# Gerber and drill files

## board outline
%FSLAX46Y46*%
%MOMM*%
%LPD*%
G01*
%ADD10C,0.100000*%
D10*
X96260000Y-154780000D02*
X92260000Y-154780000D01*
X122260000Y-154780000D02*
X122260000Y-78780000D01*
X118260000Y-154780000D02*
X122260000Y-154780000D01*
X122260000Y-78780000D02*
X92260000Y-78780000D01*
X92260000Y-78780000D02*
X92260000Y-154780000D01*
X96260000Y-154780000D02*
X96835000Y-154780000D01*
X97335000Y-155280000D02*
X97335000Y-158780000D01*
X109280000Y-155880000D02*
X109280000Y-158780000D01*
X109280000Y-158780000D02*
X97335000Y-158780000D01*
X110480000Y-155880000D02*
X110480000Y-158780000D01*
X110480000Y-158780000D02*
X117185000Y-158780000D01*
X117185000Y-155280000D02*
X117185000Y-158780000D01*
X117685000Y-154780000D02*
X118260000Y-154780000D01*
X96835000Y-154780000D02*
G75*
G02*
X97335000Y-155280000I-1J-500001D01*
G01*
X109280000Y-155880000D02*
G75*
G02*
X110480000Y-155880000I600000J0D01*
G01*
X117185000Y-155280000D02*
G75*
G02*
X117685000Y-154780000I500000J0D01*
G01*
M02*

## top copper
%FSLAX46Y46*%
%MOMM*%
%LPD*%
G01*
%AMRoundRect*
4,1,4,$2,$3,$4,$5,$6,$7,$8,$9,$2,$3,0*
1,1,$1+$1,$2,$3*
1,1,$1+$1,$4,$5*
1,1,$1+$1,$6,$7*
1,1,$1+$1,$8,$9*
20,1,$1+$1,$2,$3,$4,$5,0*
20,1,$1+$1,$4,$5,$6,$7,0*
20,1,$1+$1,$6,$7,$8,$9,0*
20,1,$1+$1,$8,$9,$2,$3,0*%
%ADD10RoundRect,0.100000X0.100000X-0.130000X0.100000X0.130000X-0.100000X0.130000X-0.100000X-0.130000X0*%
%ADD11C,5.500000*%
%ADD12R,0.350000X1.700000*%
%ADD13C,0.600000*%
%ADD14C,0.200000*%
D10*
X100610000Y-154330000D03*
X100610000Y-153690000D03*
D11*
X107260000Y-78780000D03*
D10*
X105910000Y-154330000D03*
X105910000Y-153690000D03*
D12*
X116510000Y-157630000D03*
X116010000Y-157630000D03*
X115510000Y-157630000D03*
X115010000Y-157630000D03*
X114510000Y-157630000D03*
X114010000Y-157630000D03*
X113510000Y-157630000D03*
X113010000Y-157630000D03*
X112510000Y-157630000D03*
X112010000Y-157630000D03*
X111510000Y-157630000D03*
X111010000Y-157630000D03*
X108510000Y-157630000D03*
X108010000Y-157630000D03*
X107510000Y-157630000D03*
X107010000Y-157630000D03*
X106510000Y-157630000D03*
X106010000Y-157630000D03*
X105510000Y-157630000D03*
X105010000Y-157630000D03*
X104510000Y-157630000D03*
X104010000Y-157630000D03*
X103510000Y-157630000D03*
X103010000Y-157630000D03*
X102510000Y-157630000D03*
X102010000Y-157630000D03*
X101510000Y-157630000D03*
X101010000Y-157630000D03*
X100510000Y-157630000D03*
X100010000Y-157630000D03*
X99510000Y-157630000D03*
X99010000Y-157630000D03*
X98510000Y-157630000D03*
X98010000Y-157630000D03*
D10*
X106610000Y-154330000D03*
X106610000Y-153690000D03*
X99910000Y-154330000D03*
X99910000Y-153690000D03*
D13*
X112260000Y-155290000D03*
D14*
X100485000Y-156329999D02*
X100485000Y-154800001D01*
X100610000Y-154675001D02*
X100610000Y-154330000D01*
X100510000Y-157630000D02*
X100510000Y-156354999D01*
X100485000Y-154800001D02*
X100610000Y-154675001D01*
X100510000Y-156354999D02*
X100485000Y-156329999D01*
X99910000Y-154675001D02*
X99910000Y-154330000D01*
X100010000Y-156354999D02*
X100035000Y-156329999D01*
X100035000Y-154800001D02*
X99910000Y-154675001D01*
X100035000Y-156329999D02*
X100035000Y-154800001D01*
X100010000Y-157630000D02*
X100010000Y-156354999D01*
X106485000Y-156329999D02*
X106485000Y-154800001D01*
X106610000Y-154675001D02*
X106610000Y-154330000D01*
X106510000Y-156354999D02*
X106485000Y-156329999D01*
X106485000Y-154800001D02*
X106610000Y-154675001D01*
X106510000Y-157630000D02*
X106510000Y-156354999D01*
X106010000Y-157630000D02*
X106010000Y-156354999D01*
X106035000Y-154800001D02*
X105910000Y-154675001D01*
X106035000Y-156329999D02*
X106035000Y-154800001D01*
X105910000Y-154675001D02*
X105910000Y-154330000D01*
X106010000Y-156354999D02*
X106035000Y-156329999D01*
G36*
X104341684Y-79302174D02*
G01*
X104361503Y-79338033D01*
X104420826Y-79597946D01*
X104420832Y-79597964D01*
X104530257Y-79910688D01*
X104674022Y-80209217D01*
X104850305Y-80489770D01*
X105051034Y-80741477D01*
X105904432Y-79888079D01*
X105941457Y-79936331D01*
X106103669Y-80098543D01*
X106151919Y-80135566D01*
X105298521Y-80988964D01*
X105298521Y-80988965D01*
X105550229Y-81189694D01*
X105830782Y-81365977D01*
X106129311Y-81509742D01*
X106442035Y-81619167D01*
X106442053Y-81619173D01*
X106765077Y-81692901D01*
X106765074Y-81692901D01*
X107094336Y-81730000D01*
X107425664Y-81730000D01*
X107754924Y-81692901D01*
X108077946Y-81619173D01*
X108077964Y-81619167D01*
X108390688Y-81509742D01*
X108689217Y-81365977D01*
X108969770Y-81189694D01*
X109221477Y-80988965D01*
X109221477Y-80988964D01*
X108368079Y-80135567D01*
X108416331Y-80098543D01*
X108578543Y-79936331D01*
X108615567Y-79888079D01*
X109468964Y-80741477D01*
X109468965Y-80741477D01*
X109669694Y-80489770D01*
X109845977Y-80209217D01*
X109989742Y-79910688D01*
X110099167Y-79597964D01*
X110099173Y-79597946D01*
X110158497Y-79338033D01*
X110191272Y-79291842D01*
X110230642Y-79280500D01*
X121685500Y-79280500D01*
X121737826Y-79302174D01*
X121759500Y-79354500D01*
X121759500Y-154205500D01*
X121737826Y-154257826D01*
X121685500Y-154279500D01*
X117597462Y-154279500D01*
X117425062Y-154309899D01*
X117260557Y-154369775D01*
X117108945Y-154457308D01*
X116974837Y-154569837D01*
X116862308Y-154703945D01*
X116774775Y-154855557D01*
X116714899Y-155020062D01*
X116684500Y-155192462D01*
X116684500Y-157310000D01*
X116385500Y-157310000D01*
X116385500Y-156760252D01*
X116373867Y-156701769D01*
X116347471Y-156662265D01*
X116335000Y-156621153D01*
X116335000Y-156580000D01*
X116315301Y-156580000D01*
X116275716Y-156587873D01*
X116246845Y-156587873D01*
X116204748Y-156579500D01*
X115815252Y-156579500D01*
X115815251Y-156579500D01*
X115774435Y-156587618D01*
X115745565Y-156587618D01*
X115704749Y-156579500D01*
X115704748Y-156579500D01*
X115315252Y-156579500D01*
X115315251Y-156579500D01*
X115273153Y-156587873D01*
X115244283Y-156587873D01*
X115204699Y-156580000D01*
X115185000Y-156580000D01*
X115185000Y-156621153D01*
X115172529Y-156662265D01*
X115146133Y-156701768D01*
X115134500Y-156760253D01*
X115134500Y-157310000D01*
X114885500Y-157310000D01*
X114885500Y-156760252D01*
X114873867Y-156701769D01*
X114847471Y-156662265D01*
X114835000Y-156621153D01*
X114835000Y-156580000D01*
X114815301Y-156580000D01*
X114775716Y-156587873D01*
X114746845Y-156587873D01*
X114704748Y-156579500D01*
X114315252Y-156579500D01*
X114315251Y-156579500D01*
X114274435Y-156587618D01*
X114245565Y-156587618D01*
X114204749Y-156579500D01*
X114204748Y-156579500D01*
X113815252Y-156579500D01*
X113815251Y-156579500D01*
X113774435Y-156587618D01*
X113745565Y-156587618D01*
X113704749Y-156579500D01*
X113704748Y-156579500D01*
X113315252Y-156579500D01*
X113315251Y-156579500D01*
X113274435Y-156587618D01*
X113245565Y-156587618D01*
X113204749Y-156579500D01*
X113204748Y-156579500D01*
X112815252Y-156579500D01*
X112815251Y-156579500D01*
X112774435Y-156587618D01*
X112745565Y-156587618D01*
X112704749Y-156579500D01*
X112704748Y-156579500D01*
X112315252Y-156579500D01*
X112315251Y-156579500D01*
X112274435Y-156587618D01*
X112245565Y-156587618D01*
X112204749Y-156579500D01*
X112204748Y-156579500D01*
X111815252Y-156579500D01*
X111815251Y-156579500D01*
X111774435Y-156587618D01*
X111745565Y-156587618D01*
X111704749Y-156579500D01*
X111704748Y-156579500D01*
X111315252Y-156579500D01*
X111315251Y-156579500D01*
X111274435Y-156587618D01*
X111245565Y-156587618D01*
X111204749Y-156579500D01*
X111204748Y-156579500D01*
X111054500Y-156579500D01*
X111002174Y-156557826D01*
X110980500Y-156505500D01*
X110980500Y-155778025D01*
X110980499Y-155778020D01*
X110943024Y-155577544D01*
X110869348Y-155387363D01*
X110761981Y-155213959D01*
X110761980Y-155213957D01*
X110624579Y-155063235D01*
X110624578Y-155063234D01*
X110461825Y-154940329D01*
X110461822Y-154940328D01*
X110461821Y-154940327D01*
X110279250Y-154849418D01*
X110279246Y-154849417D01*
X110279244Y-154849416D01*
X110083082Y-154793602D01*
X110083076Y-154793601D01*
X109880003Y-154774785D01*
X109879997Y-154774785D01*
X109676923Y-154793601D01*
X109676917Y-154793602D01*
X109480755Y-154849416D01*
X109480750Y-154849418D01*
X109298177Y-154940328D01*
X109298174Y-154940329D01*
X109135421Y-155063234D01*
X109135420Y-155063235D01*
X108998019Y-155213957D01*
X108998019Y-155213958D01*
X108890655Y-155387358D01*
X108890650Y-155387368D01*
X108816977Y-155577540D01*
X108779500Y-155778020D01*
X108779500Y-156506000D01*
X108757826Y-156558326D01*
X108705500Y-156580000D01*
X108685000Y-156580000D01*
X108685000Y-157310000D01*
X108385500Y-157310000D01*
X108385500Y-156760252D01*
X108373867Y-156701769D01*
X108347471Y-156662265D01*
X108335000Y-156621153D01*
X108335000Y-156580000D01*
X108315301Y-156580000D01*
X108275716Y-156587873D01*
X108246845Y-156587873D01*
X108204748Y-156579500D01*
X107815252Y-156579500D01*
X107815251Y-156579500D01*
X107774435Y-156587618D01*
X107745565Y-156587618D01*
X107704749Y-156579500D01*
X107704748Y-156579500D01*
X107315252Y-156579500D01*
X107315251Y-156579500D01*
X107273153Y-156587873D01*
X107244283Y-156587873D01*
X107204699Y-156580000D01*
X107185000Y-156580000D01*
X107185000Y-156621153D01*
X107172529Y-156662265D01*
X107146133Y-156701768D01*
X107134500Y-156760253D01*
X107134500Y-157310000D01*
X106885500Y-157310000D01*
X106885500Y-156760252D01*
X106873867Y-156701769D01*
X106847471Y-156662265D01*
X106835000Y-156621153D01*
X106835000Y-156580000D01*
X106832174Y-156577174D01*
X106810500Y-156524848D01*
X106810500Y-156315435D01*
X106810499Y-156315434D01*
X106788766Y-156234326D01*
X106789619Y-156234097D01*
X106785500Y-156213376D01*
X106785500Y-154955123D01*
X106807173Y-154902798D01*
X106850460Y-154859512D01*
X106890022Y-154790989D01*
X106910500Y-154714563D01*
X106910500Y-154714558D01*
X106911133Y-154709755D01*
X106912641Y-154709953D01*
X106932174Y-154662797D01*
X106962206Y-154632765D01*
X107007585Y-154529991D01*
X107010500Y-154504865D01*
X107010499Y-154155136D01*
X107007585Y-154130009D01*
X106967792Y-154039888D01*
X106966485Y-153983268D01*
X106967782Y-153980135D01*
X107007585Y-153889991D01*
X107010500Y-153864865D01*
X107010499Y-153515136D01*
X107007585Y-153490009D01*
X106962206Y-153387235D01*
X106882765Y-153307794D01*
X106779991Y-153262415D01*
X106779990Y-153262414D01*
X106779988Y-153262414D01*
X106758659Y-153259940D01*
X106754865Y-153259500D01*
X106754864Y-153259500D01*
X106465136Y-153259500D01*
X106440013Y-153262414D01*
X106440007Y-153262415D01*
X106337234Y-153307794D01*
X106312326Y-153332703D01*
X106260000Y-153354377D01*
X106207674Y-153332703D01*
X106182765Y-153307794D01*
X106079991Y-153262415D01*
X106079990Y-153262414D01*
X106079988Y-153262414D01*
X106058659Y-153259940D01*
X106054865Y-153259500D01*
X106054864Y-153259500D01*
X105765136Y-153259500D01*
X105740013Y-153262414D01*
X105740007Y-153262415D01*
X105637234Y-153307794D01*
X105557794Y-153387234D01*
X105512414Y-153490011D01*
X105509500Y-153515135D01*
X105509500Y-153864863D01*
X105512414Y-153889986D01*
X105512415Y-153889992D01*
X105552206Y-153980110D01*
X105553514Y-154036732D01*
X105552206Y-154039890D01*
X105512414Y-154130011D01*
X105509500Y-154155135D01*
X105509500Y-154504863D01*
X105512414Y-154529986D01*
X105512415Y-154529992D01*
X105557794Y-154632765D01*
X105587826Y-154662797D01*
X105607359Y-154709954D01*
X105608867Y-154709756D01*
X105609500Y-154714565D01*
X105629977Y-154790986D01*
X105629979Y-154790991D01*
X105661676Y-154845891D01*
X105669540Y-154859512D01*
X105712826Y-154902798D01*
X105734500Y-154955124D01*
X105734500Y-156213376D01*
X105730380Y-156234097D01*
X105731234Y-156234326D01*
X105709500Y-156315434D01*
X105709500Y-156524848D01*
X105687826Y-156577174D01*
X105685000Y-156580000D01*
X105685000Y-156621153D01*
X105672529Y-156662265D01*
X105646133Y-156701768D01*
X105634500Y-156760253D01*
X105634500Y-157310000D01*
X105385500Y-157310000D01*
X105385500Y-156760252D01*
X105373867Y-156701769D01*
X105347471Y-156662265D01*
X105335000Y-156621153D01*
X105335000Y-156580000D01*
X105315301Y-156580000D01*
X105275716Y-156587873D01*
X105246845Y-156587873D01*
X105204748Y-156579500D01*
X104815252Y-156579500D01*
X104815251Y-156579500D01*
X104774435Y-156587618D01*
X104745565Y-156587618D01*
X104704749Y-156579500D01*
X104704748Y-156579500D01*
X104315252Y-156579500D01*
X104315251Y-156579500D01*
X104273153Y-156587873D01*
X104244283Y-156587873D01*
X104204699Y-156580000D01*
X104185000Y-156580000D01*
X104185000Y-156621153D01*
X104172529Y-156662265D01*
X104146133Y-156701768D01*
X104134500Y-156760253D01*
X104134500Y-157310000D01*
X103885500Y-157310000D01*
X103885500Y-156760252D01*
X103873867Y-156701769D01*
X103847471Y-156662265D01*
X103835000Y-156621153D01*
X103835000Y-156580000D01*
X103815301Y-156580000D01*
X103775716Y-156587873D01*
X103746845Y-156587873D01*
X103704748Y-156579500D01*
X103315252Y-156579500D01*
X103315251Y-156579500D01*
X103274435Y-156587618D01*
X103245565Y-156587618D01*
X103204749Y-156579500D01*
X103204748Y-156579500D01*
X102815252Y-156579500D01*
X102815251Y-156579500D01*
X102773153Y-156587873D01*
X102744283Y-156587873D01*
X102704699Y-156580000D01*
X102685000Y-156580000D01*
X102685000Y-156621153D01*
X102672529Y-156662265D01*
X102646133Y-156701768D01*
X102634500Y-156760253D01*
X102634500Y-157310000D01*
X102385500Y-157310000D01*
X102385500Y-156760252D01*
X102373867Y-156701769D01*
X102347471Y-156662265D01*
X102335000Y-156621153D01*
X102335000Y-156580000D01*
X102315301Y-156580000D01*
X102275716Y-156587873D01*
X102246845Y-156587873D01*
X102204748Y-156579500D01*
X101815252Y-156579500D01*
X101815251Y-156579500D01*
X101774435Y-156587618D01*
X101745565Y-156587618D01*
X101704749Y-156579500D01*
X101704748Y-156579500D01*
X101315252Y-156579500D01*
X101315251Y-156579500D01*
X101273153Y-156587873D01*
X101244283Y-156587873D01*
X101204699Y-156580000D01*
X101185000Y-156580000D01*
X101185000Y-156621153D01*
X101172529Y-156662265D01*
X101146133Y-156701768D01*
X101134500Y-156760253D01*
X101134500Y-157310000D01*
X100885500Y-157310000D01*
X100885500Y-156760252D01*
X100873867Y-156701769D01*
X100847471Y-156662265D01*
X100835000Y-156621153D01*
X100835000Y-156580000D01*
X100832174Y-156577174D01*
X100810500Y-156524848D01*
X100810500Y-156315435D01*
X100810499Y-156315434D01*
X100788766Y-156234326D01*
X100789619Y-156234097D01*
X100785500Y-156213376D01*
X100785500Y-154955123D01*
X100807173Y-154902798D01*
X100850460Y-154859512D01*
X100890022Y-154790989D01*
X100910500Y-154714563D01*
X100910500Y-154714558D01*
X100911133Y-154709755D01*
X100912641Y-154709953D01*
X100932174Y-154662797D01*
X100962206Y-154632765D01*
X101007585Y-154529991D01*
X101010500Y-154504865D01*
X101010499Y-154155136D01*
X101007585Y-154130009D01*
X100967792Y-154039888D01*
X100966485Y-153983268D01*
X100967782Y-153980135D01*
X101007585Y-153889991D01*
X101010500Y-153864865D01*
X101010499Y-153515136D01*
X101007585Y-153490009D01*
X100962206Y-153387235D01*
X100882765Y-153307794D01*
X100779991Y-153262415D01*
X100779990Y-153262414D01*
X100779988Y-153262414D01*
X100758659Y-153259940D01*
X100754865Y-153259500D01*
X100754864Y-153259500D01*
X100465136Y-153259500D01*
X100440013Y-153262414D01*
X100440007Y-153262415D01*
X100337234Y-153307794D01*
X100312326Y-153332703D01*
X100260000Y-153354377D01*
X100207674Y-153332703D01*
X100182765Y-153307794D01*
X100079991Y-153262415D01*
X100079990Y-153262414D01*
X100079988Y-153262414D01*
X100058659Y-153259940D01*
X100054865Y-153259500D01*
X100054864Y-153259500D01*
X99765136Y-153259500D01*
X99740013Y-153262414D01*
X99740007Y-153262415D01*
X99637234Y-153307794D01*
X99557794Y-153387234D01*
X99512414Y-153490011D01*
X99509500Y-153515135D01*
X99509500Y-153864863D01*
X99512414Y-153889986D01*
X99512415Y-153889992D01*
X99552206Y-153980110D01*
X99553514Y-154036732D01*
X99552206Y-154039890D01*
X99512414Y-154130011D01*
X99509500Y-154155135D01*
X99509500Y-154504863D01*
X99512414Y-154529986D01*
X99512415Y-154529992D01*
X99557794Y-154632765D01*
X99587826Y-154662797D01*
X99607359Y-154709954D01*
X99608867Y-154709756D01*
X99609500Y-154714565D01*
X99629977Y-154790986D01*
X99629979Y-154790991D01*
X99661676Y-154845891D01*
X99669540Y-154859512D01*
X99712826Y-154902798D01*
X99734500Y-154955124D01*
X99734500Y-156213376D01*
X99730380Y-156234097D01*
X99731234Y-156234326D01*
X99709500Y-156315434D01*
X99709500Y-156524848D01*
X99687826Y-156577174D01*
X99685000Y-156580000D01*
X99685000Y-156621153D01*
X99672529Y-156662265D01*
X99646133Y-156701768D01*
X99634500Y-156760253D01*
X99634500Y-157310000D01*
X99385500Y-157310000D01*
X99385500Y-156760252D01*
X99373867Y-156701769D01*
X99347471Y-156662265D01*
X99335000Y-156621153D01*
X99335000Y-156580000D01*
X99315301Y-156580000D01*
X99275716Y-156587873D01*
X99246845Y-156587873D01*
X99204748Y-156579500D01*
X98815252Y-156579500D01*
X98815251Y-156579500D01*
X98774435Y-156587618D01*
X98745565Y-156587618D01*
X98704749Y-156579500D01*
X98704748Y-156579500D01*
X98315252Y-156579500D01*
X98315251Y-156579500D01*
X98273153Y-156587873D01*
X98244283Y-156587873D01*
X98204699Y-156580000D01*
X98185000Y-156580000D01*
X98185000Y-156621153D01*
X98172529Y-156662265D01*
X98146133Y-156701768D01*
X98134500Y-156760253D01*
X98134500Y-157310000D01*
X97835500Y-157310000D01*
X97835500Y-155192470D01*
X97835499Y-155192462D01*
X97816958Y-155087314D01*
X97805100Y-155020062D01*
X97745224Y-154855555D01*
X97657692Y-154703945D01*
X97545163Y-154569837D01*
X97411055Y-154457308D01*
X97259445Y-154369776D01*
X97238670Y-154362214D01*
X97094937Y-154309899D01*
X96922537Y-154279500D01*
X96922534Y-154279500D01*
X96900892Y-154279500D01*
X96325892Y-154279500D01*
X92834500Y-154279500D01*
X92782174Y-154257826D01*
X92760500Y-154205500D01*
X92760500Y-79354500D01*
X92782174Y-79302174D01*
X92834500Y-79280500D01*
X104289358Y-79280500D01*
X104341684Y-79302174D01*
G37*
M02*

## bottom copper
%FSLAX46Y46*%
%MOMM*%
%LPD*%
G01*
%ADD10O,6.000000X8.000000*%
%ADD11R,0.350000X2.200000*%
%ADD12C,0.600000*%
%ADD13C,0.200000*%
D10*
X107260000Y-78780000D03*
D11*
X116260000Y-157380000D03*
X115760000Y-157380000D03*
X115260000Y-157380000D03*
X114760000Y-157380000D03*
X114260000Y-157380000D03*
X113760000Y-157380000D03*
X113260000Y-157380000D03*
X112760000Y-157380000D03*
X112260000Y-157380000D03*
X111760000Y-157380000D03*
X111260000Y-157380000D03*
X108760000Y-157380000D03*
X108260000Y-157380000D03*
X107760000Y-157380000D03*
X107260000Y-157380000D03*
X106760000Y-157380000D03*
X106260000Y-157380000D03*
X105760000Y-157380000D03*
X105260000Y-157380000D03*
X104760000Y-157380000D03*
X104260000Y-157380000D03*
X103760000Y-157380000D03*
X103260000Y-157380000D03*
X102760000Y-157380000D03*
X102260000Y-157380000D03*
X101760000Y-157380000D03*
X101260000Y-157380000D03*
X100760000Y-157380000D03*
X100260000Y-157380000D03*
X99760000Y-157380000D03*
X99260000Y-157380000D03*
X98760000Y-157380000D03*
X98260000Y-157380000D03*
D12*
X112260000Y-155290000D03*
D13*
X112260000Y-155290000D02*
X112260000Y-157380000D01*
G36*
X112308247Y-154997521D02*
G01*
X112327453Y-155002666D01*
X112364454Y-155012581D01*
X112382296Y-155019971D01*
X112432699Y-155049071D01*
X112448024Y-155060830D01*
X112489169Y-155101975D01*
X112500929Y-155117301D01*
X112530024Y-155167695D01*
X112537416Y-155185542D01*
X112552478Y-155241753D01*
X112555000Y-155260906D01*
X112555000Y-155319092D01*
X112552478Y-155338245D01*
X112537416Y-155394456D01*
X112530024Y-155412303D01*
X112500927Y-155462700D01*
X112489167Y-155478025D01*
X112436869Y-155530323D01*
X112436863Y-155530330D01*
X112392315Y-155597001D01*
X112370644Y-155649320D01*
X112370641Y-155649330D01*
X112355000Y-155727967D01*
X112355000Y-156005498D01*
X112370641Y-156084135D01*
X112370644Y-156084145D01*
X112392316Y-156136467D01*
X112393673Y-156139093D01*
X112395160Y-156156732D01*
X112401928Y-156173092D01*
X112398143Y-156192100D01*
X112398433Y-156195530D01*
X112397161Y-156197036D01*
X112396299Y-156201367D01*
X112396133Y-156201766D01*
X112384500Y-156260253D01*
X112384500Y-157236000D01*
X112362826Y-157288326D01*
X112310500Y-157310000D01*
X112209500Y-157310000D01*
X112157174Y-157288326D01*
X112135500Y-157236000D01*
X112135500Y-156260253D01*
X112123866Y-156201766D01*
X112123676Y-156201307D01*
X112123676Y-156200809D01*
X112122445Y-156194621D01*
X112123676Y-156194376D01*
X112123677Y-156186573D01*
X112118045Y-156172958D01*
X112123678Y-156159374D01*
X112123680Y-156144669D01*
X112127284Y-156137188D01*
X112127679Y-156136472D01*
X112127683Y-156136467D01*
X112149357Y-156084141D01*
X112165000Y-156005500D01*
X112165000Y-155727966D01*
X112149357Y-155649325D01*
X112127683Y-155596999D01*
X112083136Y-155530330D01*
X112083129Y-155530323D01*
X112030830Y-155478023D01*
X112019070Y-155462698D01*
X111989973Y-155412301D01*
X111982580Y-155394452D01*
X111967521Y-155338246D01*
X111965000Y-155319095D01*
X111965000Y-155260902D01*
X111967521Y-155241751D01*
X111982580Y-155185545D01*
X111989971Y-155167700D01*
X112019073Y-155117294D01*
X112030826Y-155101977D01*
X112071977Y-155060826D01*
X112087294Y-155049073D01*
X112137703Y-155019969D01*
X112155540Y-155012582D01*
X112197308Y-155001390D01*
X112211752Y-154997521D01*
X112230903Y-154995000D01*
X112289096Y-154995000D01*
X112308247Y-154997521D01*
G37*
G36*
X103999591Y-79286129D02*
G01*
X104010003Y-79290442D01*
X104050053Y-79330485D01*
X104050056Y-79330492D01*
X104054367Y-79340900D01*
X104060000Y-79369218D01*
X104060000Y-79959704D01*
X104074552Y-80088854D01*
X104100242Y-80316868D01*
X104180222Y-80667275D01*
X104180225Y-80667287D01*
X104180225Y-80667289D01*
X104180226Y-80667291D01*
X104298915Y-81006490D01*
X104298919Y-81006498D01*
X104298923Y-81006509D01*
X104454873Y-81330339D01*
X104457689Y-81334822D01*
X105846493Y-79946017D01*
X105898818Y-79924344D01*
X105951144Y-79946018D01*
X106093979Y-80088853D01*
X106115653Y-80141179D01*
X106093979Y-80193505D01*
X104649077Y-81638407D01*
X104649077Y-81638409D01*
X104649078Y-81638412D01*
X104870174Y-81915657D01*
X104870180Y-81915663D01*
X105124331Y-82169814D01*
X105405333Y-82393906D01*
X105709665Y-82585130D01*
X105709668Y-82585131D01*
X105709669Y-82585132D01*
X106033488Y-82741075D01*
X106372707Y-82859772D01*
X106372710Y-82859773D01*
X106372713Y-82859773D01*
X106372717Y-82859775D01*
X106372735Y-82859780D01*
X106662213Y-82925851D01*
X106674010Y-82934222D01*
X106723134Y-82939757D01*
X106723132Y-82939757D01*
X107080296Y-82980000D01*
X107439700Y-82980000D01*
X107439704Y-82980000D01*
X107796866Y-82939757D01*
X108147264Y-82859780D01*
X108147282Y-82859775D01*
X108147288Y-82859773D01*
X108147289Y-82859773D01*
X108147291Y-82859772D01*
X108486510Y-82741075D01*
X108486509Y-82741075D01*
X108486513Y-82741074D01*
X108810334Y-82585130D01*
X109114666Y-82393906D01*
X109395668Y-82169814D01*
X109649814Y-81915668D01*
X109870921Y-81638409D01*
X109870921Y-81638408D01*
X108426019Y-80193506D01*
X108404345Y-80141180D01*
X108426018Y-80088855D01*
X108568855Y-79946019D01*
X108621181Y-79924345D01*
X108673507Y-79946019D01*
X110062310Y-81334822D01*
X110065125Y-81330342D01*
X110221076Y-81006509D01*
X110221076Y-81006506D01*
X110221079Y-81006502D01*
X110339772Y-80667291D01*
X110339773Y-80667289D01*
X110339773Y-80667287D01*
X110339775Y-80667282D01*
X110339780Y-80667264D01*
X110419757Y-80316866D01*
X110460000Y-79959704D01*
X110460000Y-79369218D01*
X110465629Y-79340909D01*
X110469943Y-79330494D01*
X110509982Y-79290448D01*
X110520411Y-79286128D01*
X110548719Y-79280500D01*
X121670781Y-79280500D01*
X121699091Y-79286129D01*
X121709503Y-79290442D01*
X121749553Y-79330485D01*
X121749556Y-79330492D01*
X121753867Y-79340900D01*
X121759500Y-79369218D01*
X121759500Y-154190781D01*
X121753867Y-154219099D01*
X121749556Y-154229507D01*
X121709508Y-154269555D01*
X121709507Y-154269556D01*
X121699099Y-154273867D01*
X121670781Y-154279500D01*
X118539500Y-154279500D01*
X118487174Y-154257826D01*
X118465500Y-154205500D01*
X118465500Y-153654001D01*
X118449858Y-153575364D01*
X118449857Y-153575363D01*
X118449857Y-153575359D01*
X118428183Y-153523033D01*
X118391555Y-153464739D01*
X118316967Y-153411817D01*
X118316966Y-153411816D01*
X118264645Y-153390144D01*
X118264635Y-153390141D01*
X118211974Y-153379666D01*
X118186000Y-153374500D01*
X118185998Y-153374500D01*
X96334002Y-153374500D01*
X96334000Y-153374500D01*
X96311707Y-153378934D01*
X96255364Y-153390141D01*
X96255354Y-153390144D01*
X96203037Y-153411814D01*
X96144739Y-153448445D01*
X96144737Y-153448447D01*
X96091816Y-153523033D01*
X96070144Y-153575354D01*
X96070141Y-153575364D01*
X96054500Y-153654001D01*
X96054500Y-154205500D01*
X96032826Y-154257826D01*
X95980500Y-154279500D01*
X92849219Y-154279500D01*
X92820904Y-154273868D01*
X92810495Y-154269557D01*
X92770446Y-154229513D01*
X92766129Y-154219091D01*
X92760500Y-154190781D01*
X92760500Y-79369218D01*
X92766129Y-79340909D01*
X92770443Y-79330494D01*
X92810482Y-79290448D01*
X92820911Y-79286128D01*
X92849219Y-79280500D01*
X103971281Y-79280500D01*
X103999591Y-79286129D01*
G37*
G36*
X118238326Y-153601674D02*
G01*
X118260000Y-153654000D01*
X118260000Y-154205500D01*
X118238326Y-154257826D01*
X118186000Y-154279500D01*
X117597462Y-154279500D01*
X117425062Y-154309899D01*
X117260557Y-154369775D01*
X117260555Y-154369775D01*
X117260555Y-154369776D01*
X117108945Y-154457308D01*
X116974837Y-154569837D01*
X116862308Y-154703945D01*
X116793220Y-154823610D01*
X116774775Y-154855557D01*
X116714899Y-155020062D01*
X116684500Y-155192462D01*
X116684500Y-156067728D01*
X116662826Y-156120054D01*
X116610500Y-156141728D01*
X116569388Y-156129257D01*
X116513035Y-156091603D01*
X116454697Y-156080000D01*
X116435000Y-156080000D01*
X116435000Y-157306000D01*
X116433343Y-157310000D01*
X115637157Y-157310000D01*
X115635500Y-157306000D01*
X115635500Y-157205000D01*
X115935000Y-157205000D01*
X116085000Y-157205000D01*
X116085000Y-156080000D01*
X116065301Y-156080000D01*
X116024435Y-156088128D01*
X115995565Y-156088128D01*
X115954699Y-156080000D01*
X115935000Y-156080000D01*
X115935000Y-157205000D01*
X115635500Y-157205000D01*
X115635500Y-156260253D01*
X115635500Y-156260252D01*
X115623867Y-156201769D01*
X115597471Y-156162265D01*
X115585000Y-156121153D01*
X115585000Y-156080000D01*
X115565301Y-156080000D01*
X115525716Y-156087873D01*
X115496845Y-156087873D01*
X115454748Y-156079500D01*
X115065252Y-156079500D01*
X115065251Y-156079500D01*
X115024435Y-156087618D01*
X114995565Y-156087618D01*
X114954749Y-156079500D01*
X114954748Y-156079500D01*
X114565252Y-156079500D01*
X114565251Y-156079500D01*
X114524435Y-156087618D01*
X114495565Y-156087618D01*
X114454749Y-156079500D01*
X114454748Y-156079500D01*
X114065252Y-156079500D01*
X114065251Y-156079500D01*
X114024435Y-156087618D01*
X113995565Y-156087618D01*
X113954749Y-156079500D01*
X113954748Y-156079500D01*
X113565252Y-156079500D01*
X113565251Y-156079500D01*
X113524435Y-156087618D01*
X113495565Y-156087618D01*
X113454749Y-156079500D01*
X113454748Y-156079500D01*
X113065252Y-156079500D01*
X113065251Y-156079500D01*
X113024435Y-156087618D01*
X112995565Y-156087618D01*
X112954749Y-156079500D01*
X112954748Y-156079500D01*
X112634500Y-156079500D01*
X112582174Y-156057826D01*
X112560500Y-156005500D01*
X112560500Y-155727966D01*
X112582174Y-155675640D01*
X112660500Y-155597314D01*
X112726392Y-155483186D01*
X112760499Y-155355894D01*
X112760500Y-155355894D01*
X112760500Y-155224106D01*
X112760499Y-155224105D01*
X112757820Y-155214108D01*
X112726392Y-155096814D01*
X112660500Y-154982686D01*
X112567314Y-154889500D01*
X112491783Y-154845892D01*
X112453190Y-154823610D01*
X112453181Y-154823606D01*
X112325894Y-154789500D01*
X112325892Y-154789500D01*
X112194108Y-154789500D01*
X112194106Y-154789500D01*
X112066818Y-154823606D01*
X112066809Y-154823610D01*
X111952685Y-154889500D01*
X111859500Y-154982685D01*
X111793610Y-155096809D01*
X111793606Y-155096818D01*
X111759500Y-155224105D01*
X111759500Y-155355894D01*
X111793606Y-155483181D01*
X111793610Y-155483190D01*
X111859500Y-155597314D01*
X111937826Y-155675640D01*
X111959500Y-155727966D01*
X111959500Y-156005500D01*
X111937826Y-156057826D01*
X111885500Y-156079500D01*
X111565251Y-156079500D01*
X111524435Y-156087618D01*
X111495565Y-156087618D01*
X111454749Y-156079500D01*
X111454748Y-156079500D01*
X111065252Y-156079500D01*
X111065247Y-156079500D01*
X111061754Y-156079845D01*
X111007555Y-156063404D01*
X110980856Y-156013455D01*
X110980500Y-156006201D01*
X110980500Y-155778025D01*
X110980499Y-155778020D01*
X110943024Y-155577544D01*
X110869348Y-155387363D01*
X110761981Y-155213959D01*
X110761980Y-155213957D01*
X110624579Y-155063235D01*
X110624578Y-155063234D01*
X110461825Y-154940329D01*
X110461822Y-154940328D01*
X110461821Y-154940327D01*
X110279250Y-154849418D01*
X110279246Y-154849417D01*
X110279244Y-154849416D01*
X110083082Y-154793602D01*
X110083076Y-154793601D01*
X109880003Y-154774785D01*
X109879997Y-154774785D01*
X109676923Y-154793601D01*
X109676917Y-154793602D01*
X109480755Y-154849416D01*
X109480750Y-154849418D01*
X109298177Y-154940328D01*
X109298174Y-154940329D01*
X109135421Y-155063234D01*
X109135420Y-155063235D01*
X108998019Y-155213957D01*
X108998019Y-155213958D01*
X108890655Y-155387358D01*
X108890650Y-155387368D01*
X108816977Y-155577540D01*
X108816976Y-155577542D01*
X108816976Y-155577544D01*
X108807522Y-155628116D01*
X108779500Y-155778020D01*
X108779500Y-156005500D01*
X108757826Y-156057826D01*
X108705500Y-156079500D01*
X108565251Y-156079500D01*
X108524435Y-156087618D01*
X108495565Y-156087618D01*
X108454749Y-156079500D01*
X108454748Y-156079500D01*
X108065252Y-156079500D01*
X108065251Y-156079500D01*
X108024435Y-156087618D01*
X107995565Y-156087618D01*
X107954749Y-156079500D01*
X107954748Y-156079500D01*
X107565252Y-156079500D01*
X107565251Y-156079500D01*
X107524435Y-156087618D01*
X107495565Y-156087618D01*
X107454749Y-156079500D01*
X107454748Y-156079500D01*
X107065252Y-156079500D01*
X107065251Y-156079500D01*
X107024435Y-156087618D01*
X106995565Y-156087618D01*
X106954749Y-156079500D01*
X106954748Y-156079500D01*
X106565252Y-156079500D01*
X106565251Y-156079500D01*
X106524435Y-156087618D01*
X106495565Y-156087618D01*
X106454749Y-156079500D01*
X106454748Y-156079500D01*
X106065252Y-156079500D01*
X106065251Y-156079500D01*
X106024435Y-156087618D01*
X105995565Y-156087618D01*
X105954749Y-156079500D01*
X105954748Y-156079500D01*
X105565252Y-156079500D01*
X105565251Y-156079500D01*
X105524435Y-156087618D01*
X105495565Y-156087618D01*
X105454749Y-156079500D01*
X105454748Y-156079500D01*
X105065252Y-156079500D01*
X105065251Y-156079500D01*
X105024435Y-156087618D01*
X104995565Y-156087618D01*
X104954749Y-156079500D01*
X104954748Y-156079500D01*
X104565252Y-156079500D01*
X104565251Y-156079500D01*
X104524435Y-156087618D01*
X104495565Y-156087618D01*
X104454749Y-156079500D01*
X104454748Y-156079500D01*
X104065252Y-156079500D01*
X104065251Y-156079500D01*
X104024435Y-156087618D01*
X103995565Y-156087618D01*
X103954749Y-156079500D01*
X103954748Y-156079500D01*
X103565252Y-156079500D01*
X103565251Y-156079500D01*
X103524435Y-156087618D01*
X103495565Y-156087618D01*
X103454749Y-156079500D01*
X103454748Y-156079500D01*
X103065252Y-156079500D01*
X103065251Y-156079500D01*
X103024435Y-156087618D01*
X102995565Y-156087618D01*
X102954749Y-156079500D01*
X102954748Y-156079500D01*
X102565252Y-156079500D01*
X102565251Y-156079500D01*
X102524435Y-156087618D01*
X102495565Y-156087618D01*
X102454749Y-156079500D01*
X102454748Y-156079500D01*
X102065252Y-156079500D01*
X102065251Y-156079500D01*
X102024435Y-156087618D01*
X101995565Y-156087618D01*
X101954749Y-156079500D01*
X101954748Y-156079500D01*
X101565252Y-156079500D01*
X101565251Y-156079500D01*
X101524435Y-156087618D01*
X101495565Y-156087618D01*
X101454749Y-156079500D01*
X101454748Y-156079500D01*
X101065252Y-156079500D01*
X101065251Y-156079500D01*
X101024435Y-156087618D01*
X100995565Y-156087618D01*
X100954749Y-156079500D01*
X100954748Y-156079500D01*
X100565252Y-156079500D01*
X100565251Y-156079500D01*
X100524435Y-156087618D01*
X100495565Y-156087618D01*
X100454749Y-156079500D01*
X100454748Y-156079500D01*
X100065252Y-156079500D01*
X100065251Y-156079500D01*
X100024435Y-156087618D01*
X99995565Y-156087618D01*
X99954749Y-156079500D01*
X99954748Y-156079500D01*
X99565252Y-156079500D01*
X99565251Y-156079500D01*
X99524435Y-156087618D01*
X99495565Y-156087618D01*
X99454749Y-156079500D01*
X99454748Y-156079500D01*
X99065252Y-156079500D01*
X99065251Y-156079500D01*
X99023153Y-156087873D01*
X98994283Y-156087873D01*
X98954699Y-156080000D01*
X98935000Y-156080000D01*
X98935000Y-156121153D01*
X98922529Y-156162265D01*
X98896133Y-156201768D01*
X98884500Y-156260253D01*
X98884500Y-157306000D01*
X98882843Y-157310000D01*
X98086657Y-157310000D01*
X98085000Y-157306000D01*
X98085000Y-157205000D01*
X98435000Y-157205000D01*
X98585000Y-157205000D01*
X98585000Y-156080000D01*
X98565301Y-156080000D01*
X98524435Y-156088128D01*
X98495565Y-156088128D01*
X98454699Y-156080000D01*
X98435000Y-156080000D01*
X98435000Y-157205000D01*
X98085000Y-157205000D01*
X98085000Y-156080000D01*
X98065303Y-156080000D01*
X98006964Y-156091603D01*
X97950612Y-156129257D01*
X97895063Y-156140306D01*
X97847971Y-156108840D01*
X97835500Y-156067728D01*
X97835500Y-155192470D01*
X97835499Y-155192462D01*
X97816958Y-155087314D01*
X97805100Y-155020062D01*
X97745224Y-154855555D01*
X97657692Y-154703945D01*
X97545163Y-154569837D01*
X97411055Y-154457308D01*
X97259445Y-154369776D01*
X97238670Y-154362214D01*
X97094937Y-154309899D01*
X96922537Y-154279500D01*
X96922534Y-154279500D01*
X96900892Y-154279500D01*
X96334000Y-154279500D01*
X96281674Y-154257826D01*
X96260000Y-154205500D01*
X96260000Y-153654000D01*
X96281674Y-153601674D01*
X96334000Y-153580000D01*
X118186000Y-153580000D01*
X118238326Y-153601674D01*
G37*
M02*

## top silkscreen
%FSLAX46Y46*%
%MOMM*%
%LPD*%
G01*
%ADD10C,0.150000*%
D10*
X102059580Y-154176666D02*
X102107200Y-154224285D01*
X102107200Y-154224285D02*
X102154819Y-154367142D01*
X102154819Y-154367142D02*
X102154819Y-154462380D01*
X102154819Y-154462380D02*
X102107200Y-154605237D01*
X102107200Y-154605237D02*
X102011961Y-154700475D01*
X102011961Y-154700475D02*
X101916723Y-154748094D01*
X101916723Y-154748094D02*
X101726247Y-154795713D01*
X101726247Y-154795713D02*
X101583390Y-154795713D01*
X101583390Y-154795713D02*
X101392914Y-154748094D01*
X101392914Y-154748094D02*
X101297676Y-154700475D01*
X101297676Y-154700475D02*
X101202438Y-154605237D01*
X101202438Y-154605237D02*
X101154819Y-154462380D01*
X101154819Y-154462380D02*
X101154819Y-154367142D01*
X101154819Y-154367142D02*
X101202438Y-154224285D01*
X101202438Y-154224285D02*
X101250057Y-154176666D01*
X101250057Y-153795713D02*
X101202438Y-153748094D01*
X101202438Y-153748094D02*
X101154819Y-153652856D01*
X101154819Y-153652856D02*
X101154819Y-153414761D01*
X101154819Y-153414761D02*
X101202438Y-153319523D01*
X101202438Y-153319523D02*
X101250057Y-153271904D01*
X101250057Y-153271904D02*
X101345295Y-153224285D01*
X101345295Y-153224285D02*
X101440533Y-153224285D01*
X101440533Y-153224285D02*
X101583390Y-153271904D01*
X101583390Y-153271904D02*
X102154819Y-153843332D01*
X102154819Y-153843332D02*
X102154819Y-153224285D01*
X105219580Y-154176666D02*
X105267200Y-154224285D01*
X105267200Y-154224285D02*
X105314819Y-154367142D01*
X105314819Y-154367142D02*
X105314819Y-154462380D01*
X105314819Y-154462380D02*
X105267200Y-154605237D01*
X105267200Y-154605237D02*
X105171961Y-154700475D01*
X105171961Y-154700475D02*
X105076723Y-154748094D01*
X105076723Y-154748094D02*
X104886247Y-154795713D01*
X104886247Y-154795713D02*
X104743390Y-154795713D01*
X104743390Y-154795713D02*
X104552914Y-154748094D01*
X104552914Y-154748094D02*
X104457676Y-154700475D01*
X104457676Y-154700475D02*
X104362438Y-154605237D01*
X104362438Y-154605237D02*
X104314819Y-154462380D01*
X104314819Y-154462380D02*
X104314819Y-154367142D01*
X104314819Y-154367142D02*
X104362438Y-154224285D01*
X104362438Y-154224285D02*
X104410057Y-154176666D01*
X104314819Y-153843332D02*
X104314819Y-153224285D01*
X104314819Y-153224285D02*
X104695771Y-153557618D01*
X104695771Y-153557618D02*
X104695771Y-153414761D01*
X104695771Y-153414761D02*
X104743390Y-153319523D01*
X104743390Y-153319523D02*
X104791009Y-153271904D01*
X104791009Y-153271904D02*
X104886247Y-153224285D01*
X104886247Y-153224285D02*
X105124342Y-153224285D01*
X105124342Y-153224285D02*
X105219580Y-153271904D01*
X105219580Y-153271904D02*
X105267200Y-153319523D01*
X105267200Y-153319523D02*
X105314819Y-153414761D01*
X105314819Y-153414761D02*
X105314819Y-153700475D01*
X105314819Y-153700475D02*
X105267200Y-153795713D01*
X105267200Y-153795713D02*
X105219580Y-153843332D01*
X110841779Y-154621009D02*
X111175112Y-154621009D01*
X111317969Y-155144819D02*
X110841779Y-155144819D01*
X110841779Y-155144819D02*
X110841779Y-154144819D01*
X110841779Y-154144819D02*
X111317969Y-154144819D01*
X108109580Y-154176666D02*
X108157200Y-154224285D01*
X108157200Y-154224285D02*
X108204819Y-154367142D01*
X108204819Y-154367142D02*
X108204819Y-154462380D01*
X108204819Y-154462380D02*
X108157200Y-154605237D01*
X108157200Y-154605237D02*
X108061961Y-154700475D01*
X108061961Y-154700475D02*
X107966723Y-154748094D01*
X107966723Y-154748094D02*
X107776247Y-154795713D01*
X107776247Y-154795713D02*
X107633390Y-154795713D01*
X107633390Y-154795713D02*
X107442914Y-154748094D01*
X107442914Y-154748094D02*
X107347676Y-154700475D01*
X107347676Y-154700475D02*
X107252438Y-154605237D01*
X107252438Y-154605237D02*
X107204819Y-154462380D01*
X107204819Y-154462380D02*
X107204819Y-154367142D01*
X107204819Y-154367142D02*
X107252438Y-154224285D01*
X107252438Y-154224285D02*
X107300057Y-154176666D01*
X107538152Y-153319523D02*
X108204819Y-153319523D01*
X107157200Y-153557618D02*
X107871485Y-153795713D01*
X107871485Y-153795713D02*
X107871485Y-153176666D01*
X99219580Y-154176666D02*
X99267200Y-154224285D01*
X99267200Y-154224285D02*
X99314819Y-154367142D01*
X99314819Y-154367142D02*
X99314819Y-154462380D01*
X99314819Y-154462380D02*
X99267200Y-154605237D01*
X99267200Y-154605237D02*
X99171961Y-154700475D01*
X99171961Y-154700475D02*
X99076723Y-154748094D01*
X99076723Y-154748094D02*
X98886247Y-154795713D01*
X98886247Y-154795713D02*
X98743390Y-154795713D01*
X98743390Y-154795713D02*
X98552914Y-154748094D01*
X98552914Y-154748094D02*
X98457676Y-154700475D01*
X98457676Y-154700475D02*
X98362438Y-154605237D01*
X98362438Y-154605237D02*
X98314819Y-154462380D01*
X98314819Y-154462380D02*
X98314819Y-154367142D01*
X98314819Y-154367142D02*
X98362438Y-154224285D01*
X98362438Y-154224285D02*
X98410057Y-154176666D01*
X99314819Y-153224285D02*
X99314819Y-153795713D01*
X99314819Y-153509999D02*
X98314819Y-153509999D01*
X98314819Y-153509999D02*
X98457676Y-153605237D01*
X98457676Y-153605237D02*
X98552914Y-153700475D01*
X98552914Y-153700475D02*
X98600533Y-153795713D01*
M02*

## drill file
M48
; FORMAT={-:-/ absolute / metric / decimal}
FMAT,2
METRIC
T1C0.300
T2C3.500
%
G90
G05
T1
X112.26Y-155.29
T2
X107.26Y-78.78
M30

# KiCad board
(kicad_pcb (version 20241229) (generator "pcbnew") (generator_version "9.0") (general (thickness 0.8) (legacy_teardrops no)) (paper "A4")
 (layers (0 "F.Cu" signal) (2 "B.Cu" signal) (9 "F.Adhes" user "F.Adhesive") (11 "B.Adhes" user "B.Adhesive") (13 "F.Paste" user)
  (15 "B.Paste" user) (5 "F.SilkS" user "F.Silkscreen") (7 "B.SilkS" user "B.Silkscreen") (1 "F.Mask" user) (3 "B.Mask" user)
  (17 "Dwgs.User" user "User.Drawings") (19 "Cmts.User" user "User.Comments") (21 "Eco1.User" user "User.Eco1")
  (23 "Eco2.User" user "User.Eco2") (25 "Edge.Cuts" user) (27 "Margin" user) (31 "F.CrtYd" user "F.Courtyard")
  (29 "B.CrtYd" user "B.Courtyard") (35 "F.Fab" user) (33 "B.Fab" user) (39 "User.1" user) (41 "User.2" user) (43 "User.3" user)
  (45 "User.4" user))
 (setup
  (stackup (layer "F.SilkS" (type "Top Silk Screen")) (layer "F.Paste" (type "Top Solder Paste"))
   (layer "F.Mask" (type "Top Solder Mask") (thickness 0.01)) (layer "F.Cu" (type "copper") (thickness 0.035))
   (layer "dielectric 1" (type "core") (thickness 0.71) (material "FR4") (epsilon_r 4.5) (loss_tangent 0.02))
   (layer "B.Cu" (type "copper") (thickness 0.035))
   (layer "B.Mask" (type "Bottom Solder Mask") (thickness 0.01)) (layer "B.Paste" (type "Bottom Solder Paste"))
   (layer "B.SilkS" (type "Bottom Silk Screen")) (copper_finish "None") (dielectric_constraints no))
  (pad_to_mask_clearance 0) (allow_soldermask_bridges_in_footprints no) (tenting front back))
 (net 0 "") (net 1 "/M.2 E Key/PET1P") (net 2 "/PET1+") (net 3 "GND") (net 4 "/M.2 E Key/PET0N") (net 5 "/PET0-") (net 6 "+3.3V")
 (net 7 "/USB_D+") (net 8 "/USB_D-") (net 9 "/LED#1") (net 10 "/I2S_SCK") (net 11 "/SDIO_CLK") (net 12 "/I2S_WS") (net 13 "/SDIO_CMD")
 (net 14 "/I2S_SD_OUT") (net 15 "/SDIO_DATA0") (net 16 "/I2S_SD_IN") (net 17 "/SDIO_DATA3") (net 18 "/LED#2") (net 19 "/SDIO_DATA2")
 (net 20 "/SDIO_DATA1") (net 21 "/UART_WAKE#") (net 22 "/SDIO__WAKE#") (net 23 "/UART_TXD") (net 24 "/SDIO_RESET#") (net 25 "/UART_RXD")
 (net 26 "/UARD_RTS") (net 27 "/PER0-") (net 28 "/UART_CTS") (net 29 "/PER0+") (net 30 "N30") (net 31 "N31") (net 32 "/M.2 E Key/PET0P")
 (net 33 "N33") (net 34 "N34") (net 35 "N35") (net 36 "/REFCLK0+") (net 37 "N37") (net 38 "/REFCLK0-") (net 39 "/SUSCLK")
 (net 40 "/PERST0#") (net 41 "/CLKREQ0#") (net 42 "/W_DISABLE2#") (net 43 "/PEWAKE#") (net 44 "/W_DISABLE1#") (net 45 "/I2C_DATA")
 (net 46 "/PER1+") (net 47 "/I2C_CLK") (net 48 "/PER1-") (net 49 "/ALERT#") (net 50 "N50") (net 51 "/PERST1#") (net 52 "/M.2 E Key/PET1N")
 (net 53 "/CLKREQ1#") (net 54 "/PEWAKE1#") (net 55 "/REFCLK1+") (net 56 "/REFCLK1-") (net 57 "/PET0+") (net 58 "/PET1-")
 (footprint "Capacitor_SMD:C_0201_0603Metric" (layer "F.Cu") (at 100.61 154.01 90)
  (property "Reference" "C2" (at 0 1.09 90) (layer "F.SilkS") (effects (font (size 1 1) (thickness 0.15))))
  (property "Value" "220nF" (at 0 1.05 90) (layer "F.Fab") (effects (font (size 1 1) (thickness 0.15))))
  (pad "" smd roundrect (at -0.345 0 90) (size 0.318 0.36) (layers "F.Paste") (roundrect_rratio 0.25))
  (pad "" smd roundrect (at 0.345 0 90) (size 0.318 0.36) (layers "F.Paste") (roundrect_rratio 0.25))
  (pad "1" smd roundrect (at -0.32 0 90) (size 0.46 0.4) (layers "F.Cu" "F.Mask") (roundrect_rratio 0.25) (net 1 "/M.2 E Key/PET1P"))
  (pad "2" smd roundrect (at 0.32 0 90) (size 0.46 0.4) (layers "F.Cu" "F.Mask") (roundrect_rratio 0.25) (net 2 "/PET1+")))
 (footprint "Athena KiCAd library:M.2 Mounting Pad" (layer "F.Cu") (at 107.26 78.78)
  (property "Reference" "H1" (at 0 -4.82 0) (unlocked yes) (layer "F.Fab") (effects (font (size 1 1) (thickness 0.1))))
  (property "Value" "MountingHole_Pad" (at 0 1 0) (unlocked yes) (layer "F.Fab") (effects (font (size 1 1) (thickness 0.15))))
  (pad "1" thru_hole circle (at 0 0) (size 5.5 5.5) (drill 3.5) (layers "*.Cu" "*.Mask") (remove_unused_layers no) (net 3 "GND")
   (padstack (mode front_inner_back)
    (layer "Inner" (shape circle) (size 5.5 5.5) (zone_connect -1))
    (layer "B.Cu" (shape oval) (size 6 8) (thermal_bridge_angle 45) (zone_connect -1)))))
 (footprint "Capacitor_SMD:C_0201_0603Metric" (layer "F.Cu") (at 105.91 154.01 90)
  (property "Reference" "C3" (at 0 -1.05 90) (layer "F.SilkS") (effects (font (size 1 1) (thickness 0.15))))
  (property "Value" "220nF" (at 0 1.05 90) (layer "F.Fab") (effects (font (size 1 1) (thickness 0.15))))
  (pad "" smd roundrect (at -0.345 0 90) (size 0.318 0.36) (layers "F.Paste") (roundrect_rratio 0.25))
  (pad "" smd roundrect (at 0.345 0 90) (size 0.318 0.36) (layers "F.Paste") (roundrect_rratio 0.25))
  (pad "1" smd roundrect (at -0.32 0 90) (size 0.46 0.4) (layers "F.Cu" "F.Mask") (roundrect_rratio 0.25) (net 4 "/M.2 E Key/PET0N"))
  (pad "2" smd roundrect (at 0.32 0 90) (size 0.46 0.4) (layers "F.Cu" "F.Mask") (roundrect_rratio 0.25) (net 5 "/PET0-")))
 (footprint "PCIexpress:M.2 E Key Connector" (layer "F.Cu") (at 107.26 157.67)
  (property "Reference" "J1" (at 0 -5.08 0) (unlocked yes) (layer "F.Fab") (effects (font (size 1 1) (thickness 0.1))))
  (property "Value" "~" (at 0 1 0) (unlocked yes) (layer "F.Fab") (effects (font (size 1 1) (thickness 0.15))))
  (fp_line (start -11 -2.89) (end -10.425 -2.89) (stroke (width 0.1) (type default)) (layer "Edge.Cuts") (net 1))
  (fp_line (start -9.925 -2.39) (end -9.925 1.11) (stroke (width 0.1) (type default)) (layer "Edge.Cuts") (net 1))
  (fp_line (start 2.02 -1.79) (end 2.02 1.11) (stroke (width 0.1) (type default)) (layer "Edge.Cuts") (net 1))
  (fp_line (start 2.02 1.11) (end -9.925 1.11) (stroke (width 0.1) (type default)) (layer "Edge.Cuts") (net 1))
  (fp_line (start 3.22 -1.79) (end 3.22 1.11) (stroke (width 0.1) (type default)) (layer "Edge.Cuts") (net 1))
  (fp_line (start 3.22 1.11) (end 9.925 1.11) (stroke (width 0.1) (type default)) (layer "Edge.Cuts") (net 1))
  (fp_line (start 9.925 -2.39) (end 9.925 1.11) (stroke (width 0.1) (type default)) (layer "Edge.Cuts") (net 1))
  (fp_line (start 10.425 -2.89) (end 11 -2.89) (stroke (width 0.1) (type default)) (layer "Edge.Cuts") (net 1))
  (fp_arc (start -10.425 -2.89) (mid -10.071447 -2.743553) (end -9.925 -2.39) (stroke (width 0.1) (type default)) (layer "Edge.Cuts")
   (net 1))
  (fp_arc (start 2.02 -1.79) (mid 2.62 -2.39) (end 3.22 -1.79) (stroke (width 0.1) (type default)) (layer "Edge.Cuts") (net 1))
  (fp_arc (start 9.925 -2.39) (mid 10.071447 -2.743553) (end 10.425 -2.89) (stroke (width 0.1) (type default)) (layer "Edge.Cuts") (net 1))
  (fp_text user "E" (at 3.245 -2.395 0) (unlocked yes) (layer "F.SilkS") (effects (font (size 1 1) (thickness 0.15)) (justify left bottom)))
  (pad "1" smd rect (at 9.25 -0.04 180) (size 0.35 1.7) (layers "F.Cu") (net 3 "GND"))
  (pad "2" smd rect (at 9 -0.29 180) (size 0.35 2.2) (layers "B.Cu") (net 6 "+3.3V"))
  (pad "3" smd rect (at 8.75 -0.04 180) (size 0.35 1.7) (layers "F.Cu") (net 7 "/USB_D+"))
  (pad "4" smd rect (at 8.5 -0.29 180) (size 0.35 2.2) (layers "B.Cu") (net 6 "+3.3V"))
  (pad "5" smd rect (at 8.25 -0.04 180) (size 0.35 1.7) (layers "F.Cu") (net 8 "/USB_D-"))
  (pad "6" smd rect (at 8 -0.29 180) (size 0.35 2.2) (layers "B.Cu") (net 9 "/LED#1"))
  (pad "7" smd rect (at 7.75 -0.04 180) (size 0.35 1.7) (layers "F.Cu") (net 3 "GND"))
  (pad "8" smd rect (at 7.5 -0.29 180) (size 0.35 2.2) (layers "B.Cu") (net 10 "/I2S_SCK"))
  (pad "9" smd rect (at 7.25 -0.04 180) (size 0.35 1.7) (layers "F.Cu") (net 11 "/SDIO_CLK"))
  (pad "10" smd rect (at 7 -0.29 180) (size 0.35 2.2) (layers "B.Cu") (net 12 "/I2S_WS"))
  (pad "11" smd rect (at 6.75 -0.04 180) (size 0.35 1.7) (layers "F.Cu") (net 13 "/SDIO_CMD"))
  (pad "12" smd rect (at 6.5 -0.29 180) (size 0.35 2.2) (layers "B.Cu") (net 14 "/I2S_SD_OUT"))
  (pad "13" smd rect (at 6.25 -0.04 180) (size 0.35 1.7) (layers "F.Cu") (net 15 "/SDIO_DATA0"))
  (pad "14" smd rect (at 6 -0.29 180) (size 0.35 2.2) (layers "B.Cu") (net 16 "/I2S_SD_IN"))
  (pad "15" smd rect (at 5.75 -0.04 180) (size 0.35 1.7) (layers "F.Cu") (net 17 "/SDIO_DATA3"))
  (pad "16" smd rect (at 5.5 -0.29 180) (size 0.35 2.2) (layers "B.Cu") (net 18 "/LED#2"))
  (pad "17" smd rect (at 5.25 -0.04 180) (size 0.35 1.7) (layers "F.Cu") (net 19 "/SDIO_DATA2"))
  (pad "18" smd rect (at 5 -0.29 180) (size 0.35 2.2) (layers "B.Cu") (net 3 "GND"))
  (pad "19" smd rect (at 4.75 -0.04 180) (size 0.35 1.7) (layers "F.Cu") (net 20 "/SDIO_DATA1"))
  (pad "20" smd rect (at 4.5 -0.29 180) (size 0.35 2.2) (layers "B.Cu") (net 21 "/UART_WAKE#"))
  (pad "21" smd rect (at 4.25 -0.04 180) (size 0.35 1.7) (layers "F.Cu") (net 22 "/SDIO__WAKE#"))
  (pad "22" smd rect (at 4 -0.29 180) (size 0.35 2.2) (layers "B.Cu") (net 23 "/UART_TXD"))
  (pad "23" smd rect (at 3.75 -0.04 180) (size 0.35 1.7) (layers "F.Cu") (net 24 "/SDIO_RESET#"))
  (pad "32" smd rect (at 1.5 -0.29 180) (size 0.35 2.2) (layers "B.Cu") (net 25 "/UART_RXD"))
  (pad "33" smd rect (at 1.25 -0.04 180) (size 0.35 1.7) (layers "F.Cu") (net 3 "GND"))
  (pad "34" smd rect (at 1 -0.29 180) (size 0.35 2.2) (layers "B.Cu") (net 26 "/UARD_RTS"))
  (pad "35" smd rect (at 0.75 -0.04 180) (size 0.35 1.7) (layers "F.Cu") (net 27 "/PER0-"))
  (pad "36" smd rect (at 0.5 -0.29 180) (size 0.35 2.2) (layers "B.Cu") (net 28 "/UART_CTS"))
  (pad "37" smd rect (at 0.25 -0.04 180) (size 0.35 1.7) (layers "F.Cu") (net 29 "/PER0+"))
  (pad "38" smd rect (at 0 -0.29 180) (size 0.35 2.2) (layers "B.Cu") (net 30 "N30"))
  (pad "39" smd rect (at -0.25 -0.04 180) (size 0.35 1.7) (layers "F.Cu") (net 3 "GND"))
  (pad "40" smd rect (at -0.5 -0.29 180) (size 0.35 2.2) (layers "B.Cu") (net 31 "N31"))
  (pad "41" smd rect (at -0.75 -0.04 180) (size 0.35 1.7) (layers "F.Cu") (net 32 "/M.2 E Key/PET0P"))
  (pad "42" smd rect (at -1 -0.29 180) (size 0.35 2.2) (layers "B.Cu") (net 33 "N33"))
  (pad "43" smd rect (at -1.25 -0.04 180) (size 0.35 1.7) (layers "F.Cu") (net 4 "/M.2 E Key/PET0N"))
  (pad "44" smd rect (at -1.5 -0.29 180) (size 0.35 2.2) (layers "B.Cu") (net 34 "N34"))
  (pad "45" smd rect (at -1.75 -0.04 180) (size 0.35 1.7) (layers "F.Cu") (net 3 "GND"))
  (pad "46" smd rect (at -2 -0.29 180) (size 0.35 2.2) (layers "B.Cu") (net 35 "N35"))
  (pad "47" smd rect (at -2.25 -0.04 180) (size 0.35 1.7) (layers "F.Cu") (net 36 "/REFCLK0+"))
  (pad "48" smd rect (at -2.5 -0.29 180) (size 0.35 2.2) (layers "B.Cu") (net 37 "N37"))
  (pad "49" smd rect (at -2.75 -0.04 180) (size 0.35 1.7) (layers "F.Cu") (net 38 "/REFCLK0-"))
  (pad "50" smd rect (at -3 -0.29 180) (size 0.35 2.2) (layers "B.Cu") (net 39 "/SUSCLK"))
  (pad "51" smd rect (at -3.25 -0.04 180) (size 0.35 1.7) (layers "F.Cu") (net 3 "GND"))
  (pad "52" smd rect (at -3.5 -0.29 180) (size 0.35 2.2) (layers "B.Cu") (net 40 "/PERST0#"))
  (pad "53" smd rect (at -3.75 -0.04 180) (size 0.35 1.7) (layers "F.Cu") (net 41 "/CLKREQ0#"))
  (pad "54" smd rect (at -4 -0.29 180) (size 0.35 2.2) (layers "B.Cu") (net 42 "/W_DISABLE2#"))
  (pad "55" smd rect (at -4.25 -0.04 180) (size 0.35 1.7) (layers "F.Cu") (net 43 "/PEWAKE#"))
  (pad "56" smd rect (at -4.5 -0.29 180) (size 0.35 2.2) (layers "B.Cu") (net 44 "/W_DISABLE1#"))
  (pad "57" smd rect (at -4.75 -0.04 180) (size 0.35 1.7) (layers "F.Cu") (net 3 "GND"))
  (pad "58" smd rect (at -5 -0.29 180) (size 0.35 2.2) (layers "B.Cu") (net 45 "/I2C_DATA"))
  (pad "59" smd rect (at -5.25 -0.04 180) (size 0.35 1.7) (layers "F.Cu") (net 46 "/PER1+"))
  (pad "60" smd rect (at -5.5 -0.29 180) (size 0.35 2.2) (layers "B.Cu") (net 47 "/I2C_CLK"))
  (pad "61" smd rect (at -5.75 -0.04 180) (size 0.35 1.7) (layers "F.Cu") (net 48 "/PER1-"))
  (pad "62" smd rect (at -6 -0.29 180) (size 0.35 2.2) (layers "B.Cu") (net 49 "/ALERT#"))
  (pad "63" smd rect (at -6.25 -0.04 180) (size 0.35 1.7) (layers "F.Cu") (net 3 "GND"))
  (pad "64" smd rect (at -6.5 -0.29 180) (size 0.35 2.2) (layers "B.Cu") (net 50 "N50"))
  (pad "65" smd rect (at -6.75 -0.04 180) (size 0.35 1.7) (layers "F.Cu") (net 1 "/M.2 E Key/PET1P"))
  (pad "66" smd rect (at -7 -0.29 180) (size 0.35 2.2) (layers "B.Cu") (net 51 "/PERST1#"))
  (pad "67" smd rect (at -7.25 -0.04 180) (size 0.35 1.7) (layers "F.Cu") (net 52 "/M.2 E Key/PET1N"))
  (pad "68" smd rect (at -7.5 -0.29 180) (size 0.35 2.2) (layers "B.Cu") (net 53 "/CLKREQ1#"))
  (pad "69" smd rect (at -7.75 -0.04 180) (size 0.35 1.7) (layers "F.Cu") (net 3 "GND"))
  (pad "70" smd rect (at -8 -0.29 180) (size 0.35 2.2) (layers "B.Cu") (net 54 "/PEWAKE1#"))
  (pad "71" smd rect (at -8.25 -0.04 180) (size 0.35 1.7) (layers "F.Cu") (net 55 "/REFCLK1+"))
  (pad "72" smd rect (at -8.5 -0.29 180) (size 0.35 2.2) (layers "B.Cu") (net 6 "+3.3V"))
  (pad "73" smd rect (at -8.75 -0.04 180) (size 0.35 1.7) (layers "F.Cu") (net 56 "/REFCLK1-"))
  (pad "74" smd rect (at -9 -0.29 180) (size 0.35 2.2) (layers "B.Cu") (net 6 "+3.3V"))
  (pad "75" smd rect (at -9.25 -0.04 180) (size 0.35 1.7) (layers "F.Cu") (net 3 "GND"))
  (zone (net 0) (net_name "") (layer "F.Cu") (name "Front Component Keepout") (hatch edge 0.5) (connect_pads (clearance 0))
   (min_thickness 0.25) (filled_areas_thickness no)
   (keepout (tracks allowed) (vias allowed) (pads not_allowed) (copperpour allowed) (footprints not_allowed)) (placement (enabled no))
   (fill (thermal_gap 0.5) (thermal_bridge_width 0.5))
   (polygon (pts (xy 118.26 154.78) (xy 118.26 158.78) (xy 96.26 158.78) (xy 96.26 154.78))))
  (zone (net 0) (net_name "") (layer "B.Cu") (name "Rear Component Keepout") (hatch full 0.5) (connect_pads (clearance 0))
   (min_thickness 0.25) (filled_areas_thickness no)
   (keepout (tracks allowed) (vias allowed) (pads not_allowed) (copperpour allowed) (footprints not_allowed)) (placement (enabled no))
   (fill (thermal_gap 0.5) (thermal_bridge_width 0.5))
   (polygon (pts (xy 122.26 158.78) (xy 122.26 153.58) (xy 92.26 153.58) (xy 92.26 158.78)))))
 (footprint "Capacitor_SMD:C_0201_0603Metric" (layer "F.Cu") (at 106.61 154.01 90)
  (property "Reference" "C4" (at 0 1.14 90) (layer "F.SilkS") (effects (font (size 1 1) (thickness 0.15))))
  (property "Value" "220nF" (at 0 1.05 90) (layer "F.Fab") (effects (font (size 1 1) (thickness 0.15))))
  (pad "" smd roundrect (at -0.345 0 90) (size 0.318 0.36) (layers "F.Paste") (roundrect_rratio 0.25))
  (pad "" smd roundrect (at 0.345 0 90) (size 0.318 0.36) (layers "F.Paste") (roundrect_rratio 0.25))
  (pad "1" smd roundrect (at -0.32 0 90) (size 0.46 0.4) (layers "F.Cu" "F.Mask") (roundrect_rratio 0.25) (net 32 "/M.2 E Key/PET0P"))
  (pad "2" smd roundrect (at 0.32 0 90) (size 0.46 0.4) (layers "F.Cu" "F.Mask") (roundrect_rratio 0.25) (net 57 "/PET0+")))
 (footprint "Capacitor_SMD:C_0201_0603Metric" (layer "F.Cu") (at 99.91 154.01 90)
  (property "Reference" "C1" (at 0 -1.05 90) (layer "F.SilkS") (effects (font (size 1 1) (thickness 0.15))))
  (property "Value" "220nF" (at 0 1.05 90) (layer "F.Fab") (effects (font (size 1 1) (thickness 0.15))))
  (pad "" smd roundrect (at -0.345 0 90) (size 0.318 0.36) (layers "F.Paste") (roundrect_rratio 0.25))
  (pad "" smd roundrect (at 0.345 0 90) (size 0.318 0.36) (layers "F.Paste") (roundrect_rratio 0.25))
  (pad "1" smd roundrect (at -0.32 0 90) (size 0.46 0.4) (layers "F.Cu" "F.Mask") (roundrect_rratio 0.25) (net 52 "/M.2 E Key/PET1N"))
  (pad "2" smd roundrect (at 0.32 0 90) (size 0.46 0.4) (layers "F.Cu" "F.Mask") (roundrect_rratio 0.25) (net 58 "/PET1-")))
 (gr_line (start 96.26 154.78) (end 92.26 154.78) (stroke (width 0.1) (type default)) (layer "Edge.Cuts"))
 (gr_line (start 122.26 154.78) (end 122.26 78.78) (stroke (width 0.1) (type default)) (layer "Edge.Cuts"))
 (gr_line (start 118.26 154.78) (end 122.26 154.78) (stroke (width 0.1) (type default)) (layer "Edge.Cuts"))
 (gr_line (start 122.26 78.78) (end 92.26 78.78) (stroke (width 0.1) (type default)) (layer "Edge.Cuts"))
 (gr_line (start 92.26 78.78) (end 92.26 154.78) (stroke (width 0.1) (type default)) (layer "Edge.Cuts"))
 (segment (start 100.485 156.329999) (end 100.485 154.800001) (width 0.2) (layer "F.Cu") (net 1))
 (segment (start 100.61 154.675001) (end 100.61 154.33) (width 0.2) (layer "F.Cu") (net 1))
 (segment (start 100.51 157.63) (end 100.51 156.354999) (width 0.2) (layer "F.Cu") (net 1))
 (segment (start 100.485 154.800001) (end 100.61 154.675001) (width 0.2) (layer "F.Cu") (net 1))
 (segment (start 100.51 156.354999) (end 100.485 156.329999) (width 0.2) (layer "F.Cu") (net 1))
 (segment (start 99.91 154.675001) (end 99.91 154.33) (width 0.2) (layer "F.Cu") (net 52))
 (segment (start 100.01 156.354999) (end 100.035 156.329999) (width 0.2) (layer "F.Cu") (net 52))
 (segment (start 100.035 154.800001) (end 99.91 154.675001) (width 0.2) (layer "F.Cu") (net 52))
 (segment (start 100.035 156.329999) (end 100.035 154.800001) (width 0.2) (layer "F.Cu") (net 52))
 (segment (start 100.01 157.63) (end 100.01 156.354999) (width 0.2) (layer "F.Cu") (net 52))
 (segment (start 106.485 156.329999) (end 106.485 154.800001) (width 0.2) (layer "F.Cu") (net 32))
 (segment (start 106.61 154.675001) (end 106.61 154.33) (width 0.2) (layer "F.Cu") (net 32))
 (segment (start 106.51 156.354999) (end 106.485 156.329999) (width 0.2) (layer "F.Cu") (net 32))
 (segment (start 106.485 154.800001) (end 106.61 154.675001) (width 0.2) (layer "F.Cu") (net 32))
 (segment (start 106.51 157.63) (end 106.51 156.354999) (width 0.2) (layer "F.Cu") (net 32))
 (segment (start 106.01 157.63) (end 106.01 156.354999) (width 0.2) (layer "F.Cu") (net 4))
 (segment (start 106.035 154.800001) (end 105.91 154.675001) (width 0.2) (layer "F.Cu") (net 4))
 (segment (start 106.035 156.329999) (end 106.035 154.800001) (width 0.2) (layer "F.Cu") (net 4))
 (segment (start 105.91 154.675001) (end 105.91 154.33) (width 0.2) (layer "F.Cu") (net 4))
 (segment (start 106.01 156.354999) (end 106.035 156.329999) (width 0.2) (layer "F.Cu") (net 4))
 (via (at 112.26 155.29) (size 0.6) (drill 0.3) (layers "F.Cu" "B.Cu") (free yes) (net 3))
 (segment (start 112.26 155.29) (end 112.26 157.38) (width 0.2) (layer "B.Cu") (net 3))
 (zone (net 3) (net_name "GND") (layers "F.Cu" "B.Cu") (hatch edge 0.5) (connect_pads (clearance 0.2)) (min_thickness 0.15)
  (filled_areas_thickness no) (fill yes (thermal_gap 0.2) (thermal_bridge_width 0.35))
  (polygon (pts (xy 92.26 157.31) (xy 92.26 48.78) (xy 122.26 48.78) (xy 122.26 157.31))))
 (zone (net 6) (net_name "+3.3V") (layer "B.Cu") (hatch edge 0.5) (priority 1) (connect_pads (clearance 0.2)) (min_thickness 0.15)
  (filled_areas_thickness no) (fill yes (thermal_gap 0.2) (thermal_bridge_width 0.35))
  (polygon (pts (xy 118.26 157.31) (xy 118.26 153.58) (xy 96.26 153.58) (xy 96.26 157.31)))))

